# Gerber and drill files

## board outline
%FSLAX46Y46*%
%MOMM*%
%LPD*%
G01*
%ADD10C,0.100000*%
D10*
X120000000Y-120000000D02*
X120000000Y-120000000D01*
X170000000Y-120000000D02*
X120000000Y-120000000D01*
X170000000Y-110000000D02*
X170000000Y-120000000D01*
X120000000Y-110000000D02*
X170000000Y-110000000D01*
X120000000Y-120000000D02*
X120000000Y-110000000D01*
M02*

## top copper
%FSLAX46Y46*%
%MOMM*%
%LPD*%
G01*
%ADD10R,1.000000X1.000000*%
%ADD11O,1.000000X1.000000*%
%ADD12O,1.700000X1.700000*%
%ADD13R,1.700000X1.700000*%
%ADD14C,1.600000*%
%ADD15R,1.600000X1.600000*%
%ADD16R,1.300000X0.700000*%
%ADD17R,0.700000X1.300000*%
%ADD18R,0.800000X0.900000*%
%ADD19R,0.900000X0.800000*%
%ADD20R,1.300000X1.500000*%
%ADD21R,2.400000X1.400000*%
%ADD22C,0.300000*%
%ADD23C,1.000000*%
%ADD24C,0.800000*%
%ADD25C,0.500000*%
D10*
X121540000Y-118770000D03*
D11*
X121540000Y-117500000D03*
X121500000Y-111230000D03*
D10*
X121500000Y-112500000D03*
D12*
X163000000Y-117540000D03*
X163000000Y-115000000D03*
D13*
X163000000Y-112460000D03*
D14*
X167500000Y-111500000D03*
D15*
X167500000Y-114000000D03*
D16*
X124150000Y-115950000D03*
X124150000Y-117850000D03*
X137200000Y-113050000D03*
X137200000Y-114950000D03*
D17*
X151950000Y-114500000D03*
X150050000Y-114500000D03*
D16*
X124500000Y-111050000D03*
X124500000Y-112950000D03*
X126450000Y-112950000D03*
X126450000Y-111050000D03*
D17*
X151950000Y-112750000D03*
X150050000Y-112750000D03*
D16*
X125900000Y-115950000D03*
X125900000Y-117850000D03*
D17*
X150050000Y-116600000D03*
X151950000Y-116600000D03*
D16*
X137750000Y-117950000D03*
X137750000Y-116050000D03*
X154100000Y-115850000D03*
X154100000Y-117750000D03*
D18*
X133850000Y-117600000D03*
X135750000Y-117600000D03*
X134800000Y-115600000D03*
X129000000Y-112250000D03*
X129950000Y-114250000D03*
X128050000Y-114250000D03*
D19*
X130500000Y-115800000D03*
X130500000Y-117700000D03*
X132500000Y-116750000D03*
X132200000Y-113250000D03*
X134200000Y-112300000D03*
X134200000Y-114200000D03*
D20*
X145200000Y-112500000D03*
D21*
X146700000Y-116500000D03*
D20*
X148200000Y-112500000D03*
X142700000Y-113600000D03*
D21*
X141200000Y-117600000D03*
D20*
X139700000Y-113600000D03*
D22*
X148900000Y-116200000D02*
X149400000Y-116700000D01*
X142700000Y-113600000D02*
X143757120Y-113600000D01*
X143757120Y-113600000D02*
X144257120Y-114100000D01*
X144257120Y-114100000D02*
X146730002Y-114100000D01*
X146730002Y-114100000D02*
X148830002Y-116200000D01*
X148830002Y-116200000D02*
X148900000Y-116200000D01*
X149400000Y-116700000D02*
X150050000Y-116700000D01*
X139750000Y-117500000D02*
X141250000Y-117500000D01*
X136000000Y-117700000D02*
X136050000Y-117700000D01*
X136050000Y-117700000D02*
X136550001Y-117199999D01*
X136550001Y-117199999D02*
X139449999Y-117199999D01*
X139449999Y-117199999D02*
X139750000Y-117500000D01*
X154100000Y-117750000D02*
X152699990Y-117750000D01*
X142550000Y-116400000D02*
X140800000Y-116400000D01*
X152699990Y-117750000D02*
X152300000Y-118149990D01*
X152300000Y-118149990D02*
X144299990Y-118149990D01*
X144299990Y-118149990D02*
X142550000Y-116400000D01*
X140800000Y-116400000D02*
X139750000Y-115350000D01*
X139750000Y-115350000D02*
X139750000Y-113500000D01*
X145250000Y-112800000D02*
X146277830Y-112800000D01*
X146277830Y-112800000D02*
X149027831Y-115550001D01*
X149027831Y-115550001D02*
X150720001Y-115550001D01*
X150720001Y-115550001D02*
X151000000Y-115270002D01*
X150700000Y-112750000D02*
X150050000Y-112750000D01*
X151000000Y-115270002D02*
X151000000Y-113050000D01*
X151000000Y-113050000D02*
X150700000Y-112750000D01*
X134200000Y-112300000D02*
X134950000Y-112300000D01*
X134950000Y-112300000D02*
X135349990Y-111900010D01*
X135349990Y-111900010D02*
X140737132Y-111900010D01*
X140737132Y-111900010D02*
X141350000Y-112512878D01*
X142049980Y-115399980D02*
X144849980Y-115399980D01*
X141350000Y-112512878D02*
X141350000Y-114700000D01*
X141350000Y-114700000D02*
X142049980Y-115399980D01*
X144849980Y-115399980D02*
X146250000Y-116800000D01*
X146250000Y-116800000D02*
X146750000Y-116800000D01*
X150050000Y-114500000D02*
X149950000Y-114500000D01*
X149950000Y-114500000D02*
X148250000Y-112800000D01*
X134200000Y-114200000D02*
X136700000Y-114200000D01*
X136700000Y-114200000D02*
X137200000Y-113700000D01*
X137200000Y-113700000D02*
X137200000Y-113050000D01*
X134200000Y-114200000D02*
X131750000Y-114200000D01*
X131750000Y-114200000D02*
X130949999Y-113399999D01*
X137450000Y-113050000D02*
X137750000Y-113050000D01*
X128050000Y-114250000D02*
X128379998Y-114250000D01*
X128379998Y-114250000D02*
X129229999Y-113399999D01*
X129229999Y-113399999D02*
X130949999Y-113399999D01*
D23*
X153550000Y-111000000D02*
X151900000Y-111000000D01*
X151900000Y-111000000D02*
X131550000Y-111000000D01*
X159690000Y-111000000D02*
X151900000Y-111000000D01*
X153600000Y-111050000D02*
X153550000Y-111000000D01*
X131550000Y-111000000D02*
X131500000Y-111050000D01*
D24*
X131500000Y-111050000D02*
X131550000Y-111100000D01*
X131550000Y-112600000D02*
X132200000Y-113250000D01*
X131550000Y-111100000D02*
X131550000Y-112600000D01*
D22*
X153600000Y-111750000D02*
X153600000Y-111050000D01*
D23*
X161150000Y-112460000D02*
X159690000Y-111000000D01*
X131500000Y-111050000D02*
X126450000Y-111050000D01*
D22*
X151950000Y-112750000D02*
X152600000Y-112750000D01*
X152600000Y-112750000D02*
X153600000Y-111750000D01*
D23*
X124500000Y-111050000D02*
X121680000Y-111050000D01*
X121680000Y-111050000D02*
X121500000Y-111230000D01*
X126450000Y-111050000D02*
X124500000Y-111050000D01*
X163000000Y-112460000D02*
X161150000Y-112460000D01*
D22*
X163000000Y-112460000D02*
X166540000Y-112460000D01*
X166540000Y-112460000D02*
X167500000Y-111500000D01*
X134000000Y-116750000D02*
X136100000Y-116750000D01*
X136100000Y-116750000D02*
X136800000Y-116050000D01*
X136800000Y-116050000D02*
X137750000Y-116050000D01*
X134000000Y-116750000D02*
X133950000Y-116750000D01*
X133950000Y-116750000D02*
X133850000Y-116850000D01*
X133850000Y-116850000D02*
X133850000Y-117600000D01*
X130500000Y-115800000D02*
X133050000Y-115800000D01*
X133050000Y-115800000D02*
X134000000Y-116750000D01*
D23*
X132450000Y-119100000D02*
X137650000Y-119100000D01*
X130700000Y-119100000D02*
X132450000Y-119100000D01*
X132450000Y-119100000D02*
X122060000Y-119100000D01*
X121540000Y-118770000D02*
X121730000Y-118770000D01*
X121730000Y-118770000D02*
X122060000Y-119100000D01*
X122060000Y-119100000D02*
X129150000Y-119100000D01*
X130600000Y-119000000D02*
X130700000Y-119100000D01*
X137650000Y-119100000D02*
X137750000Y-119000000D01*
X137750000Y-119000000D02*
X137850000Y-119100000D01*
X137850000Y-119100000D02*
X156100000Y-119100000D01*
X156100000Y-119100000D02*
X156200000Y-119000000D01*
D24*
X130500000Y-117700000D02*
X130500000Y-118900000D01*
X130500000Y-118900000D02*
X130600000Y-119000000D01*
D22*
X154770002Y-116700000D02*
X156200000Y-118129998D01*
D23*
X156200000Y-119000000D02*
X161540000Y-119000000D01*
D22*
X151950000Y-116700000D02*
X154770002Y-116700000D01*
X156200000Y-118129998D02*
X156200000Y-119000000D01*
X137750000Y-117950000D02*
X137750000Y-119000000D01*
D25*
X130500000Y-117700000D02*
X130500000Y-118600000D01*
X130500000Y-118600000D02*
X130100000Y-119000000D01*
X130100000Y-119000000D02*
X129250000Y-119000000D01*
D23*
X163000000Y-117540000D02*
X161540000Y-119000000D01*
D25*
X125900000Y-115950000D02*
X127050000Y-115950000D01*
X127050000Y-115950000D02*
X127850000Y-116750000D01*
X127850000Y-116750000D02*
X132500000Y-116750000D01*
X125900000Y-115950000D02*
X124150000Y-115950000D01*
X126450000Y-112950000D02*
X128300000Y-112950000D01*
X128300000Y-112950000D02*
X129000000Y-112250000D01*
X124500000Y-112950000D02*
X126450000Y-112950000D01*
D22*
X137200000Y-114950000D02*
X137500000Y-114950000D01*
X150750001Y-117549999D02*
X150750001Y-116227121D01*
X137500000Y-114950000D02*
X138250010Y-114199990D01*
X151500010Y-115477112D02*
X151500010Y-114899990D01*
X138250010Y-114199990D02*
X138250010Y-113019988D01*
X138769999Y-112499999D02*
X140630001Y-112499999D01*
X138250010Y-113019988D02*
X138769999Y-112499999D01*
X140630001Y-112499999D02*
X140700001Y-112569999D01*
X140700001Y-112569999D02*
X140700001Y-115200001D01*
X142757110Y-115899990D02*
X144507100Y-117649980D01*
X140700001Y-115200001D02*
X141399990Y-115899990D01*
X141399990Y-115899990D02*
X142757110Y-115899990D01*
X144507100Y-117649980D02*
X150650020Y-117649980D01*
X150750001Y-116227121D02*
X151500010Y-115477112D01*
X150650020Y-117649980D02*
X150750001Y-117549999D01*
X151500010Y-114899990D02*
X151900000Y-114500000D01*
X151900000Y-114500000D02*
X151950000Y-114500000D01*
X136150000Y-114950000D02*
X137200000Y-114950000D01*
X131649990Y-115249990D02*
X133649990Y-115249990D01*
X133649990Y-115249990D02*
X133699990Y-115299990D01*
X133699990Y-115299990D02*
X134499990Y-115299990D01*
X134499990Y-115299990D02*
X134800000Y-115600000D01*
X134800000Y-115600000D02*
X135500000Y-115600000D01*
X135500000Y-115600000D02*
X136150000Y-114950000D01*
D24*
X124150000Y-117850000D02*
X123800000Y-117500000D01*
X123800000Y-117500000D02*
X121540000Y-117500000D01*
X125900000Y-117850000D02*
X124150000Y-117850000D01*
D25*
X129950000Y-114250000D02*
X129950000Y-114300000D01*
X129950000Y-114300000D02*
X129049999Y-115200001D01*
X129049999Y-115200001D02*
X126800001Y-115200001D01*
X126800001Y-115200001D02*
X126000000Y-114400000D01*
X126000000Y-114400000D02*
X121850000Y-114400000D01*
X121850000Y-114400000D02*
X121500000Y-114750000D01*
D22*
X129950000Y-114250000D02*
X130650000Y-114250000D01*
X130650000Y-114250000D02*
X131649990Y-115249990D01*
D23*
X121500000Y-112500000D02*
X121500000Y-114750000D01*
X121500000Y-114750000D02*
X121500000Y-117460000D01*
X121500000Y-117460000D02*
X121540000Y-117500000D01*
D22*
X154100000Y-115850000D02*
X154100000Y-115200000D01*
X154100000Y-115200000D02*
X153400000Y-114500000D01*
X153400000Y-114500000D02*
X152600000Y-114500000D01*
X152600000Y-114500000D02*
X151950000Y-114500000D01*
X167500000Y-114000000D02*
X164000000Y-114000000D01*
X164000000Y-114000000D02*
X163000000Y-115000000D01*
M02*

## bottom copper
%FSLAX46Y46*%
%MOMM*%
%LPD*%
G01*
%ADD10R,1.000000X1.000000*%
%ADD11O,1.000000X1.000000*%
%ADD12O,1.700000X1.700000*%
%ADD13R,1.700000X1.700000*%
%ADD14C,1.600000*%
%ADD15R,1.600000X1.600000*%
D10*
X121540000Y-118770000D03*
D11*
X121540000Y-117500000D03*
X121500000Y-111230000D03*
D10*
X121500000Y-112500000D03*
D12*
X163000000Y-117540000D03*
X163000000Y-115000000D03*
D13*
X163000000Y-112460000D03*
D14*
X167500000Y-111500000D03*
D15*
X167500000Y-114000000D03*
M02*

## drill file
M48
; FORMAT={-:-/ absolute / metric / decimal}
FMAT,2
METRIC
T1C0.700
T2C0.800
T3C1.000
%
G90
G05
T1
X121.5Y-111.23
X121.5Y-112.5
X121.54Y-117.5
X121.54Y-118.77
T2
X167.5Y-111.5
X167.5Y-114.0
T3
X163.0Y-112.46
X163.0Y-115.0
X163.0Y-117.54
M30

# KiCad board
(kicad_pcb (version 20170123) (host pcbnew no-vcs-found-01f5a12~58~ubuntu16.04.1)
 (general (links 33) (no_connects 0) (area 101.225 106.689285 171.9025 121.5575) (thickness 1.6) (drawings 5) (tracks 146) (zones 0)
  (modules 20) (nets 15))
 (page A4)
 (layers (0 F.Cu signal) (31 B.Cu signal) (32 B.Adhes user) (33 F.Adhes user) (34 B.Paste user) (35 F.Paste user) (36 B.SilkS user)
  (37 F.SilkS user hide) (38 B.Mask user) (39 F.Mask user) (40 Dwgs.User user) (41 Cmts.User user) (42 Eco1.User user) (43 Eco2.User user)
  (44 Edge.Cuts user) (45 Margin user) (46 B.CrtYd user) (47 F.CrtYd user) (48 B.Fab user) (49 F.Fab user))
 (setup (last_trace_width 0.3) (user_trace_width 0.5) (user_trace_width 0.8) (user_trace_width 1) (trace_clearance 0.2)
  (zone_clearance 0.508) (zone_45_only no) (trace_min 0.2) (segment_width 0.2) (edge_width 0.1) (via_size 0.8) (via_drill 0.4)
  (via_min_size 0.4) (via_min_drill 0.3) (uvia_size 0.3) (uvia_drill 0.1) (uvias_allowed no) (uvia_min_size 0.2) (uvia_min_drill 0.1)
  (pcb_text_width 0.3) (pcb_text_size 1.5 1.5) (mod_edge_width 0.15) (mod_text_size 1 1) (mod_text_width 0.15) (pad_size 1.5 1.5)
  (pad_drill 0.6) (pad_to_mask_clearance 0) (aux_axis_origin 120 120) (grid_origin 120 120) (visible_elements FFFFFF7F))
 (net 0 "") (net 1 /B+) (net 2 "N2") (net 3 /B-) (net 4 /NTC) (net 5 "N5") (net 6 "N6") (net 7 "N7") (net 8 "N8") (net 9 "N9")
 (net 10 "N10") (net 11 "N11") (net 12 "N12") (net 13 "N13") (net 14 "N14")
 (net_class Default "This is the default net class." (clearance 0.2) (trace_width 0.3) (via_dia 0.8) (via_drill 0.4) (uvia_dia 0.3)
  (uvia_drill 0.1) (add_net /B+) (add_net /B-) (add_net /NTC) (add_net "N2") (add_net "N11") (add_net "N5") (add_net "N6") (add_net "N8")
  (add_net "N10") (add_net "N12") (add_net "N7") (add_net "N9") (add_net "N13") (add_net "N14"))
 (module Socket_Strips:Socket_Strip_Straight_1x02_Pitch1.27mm (layer F.Cu) (at 121.54 118.77 180)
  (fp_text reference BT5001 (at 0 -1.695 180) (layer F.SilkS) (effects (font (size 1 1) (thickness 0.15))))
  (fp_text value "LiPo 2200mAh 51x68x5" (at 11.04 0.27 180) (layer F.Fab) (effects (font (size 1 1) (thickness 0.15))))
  (pad 1 thru_hole rect (at 0 0 180) (size 1 1) (drill 0.7) (layers *.Cu *.Mask) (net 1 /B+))
  (pad 2 thru_hole oval (at 0 1.27 180) (size 1 1) (drill 0.7) (layers *.Cu *.Mask) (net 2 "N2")))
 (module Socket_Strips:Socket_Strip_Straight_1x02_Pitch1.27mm (layer F.Cu) (at 121.5 112.5 180)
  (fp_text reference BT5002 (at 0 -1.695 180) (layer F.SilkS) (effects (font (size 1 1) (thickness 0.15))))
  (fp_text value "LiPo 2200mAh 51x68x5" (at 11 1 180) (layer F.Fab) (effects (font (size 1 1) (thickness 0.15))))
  (pad 2 thru_hole oval (at 0 1.27 180) (size 1 1) (drill 0.7) (layers *.Cu *.Mask) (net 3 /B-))
  (pad 1 thru_hole rect (at 0 0 180) (size 1 1) (drill 0.7) (layers *.Cu *.Mask) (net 2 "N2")))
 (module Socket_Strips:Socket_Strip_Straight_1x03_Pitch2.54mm (layer F.Cu) (at 163 112.46)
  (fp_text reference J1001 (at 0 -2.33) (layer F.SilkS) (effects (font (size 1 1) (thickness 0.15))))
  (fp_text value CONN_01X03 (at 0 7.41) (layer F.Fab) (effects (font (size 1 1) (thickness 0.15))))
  (pad 3 thru_hole oval (at 0 5.08) (size 1.7 1.7) (drill 1) (layers *.Cu *.Mask) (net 1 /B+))
  (pad 2 thru_hole oval (at 0 2.54) (size 1.7 1.7) (drill 1) (layers *.Cu *.Mask) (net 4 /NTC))
  (pad 1 thru_hole rect (at 0 0) (size 1.7 1.7) (drill 1) (layers *.Cu *.Mask) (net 3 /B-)))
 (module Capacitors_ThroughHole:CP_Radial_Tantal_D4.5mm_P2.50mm (layer F.Cu) (at 167.5 114 90)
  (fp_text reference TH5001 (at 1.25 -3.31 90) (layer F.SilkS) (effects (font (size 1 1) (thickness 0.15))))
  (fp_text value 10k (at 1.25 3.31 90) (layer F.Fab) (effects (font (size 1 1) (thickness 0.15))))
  (pad 2 thru_hole circle (at 2.5 0 90) (size 1.6 1.6) (drill 0.8) (layers *.Cu *.Mask) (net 3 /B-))
  (pad 1 thru_hole rect (at 0 0 90) (size 1.6 1.6) (drill 0.8) (layers *.Cu *.Mask) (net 4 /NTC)))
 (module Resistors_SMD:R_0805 (layer F.Cu) (at 124.15 116.9 270)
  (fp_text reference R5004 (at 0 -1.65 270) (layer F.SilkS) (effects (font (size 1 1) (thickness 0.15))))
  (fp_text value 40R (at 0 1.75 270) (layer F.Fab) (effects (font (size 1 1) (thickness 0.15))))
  (pad 1 smd rect (at -0.95 0 270) (size 0.7 1.3) (layers F.Cu F.Paste F.Mask) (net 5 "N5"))
  (pad 2 smd rect (at 0.95 0 270) (size 0.7 1.3) (layers F.Cu F.Paste F.Mask) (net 2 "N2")))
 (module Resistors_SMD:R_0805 (layer F.Cu) (at 137.2 114 90)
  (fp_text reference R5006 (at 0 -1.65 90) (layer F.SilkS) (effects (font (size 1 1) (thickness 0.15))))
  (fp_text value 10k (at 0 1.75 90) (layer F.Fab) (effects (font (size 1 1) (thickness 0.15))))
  (pad 2 smd rect (at 0.95 0 90) (size 0.7 1.3) (layers F.Cu F.Paste F.Mask) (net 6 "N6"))
  (pad 1 smd rect (at -0.95 0 90) (size 0.7 1.3) (layers F.Cu F.Paste F.Mask) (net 2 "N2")))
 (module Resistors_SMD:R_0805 (layer F.Cu) (at 151 114.5 180)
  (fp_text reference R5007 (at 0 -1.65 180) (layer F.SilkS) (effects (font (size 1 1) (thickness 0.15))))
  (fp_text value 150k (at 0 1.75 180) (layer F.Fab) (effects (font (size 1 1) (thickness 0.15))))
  (pad 1 smd rect (at -0.95 0 180) (size 0.7 1.3) (layers F.Cu F.Paste F.Mask) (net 2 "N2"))
  (pad 2 smd rect (at 0.95 0 180) (size 0.7 1.3) (layers F.Cu F.Paste F.Mask) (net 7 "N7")))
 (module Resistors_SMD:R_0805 (layer F.Cu) (at 124.5 112 90)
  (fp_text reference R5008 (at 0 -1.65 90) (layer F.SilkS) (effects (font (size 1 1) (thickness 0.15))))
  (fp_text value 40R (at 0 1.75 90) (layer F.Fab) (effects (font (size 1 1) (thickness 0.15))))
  (pad 2 smd rect (at 0.95 0 90) (size 0.7 1.3) (layers F.Cu F.Paste F.Mask) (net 3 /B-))
  (pad 1 smd rect (at -0.95 0 90) (size 0.7 1.3) (layers F.Cu F.Paste F.Mask) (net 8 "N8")))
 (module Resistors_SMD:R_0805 (layer F.Cu) (at 126.45 112 90)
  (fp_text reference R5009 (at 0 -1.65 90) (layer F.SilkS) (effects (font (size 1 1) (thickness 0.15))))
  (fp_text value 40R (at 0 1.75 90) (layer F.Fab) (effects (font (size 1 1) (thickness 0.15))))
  (pad 1 smd rect (at -0.95 0 90) (size 0.7 1.3) (layers F.Cu F.Paste F.Mask) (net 8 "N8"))
  (pad 2 smd rect (at 0.95 0 90) (size 0.7 1.3) (layers F.Cu F.Paste F.Mask) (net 3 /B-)))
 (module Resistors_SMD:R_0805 (layer F.Cu) (at 151 112.75)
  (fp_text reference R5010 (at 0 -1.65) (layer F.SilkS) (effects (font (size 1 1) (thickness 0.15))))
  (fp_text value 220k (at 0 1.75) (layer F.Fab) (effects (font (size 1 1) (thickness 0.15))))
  (pad 2 smd rect (at 0.95 0) (size 0.7 1.3) (layers F.Cu F.Paste F.Mask) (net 3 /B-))
  (pad 1 smd rect (at -0.95 0) (size 0.7 1.3) (layers F.Cu F.Paste F.Mask) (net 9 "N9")))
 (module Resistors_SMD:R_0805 (layer F.Cu) (at 125.9 116.9 270)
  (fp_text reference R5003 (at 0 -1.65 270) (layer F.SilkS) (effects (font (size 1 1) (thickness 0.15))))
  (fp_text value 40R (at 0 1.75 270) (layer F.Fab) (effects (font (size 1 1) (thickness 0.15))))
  (pad 1 smd rect (at -0.95 0 270) (size 0.7 1.3) (layers F.Cu F.Paste F.Mask) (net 5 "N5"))
  (pad 2 smd rect (at 0.95 0 270) (size 0.7 1.3) (layers F.Cu F.Paste F.Mask) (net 2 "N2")))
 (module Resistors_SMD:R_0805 (layer F.Cu) (at 151 116.6 180)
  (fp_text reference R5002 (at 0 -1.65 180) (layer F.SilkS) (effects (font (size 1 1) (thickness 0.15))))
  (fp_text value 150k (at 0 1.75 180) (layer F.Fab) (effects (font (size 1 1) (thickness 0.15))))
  (pad 2 smd rect (at 0.95 0 180) (size 0.7 1.3) (layers F.Cu F.Paste F.Mask) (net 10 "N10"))
  (pad 1 smd rect (at -0.95 0 180) (size 0.7 1.3) (layers F.Cu F.Paste F.Mask) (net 1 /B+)))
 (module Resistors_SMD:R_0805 (layer F.Cu) (at 137.75 117 90)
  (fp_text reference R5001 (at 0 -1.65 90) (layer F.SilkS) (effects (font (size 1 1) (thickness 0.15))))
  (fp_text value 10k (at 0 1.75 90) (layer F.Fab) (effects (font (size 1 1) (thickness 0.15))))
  (pad 1 smd rect (at -0.95 0 90) (size 0.7 1.3) (layers F.Cu F.Paste F.Mask) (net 1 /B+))
  (pad 2 smd rect (at 0.95 0 90) (size 0.7 1.3) (layers F.Cu F.Paste F.Mask) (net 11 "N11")))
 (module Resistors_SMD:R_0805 (layer F.Cu) (at 154.1 116.8 90)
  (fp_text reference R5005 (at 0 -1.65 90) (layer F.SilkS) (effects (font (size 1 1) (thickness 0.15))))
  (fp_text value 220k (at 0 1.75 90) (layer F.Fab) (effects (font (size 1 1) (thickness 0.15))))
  (pad 2 smd rect (at 0.95 0 90) (size 0.7 1.3) (layers F.Cu F.Paste F.Mask) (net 2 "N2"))
  (pad 1 smd rect (at -0.95 0 90) (size 0.7 1.3) (layers F.Cu F.Paste F.Mask) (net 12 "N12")))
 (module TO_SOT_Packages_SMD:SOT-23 (layer F.Cu) (at 134.8 116.6 90)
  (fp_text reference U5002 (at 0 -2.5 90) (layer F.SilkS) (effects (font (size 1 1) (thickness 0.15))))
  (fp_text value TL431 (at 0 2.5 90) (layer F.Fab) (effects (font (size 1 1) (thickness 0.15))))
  (pad 1 smd rect (at -1 -0.95 90) (size 0.9 0.8) (layers F.Cu F.Paste F.Mask) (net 11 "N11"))
  (pad 2 smd rect (at -1 0.95 90) (size 0.9 0.8) (layers F.Cu F.Paste F.Mask) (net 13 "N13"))
  (pad 3 smd rect (at 1 0 90) (size 0.9 0.8) (layers F.Cu F.Paste F.Mask) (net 2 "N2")))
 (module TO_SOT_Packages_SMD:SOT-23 (layer F.Cu) (at 129 113.25 90)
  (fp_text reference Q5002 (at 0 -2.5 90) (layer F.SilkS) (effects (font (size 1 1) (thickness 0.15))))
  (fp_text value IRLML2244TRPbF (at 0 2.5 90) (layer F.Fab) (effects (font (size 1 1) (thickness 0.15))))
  (pad 3 smd rect (at 1 0 90) (size 0.9 0.8) (layers F.Cu F.Paste F.Mask) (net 8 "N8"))
  (pad 2 smd rect (at -1 0.95 90) (size 0.9 0.8) (layers F.Cu F.Paste F.Mask) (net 2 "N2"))
  (pad 1 smd rect (at -1 -0.95 90) (size 0.9 0.8) (layers F.Cu F.Paste F.Mask) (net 6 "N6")))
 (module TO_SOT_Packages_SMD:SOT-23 (layer F.Cu) (at 131.5 116.75)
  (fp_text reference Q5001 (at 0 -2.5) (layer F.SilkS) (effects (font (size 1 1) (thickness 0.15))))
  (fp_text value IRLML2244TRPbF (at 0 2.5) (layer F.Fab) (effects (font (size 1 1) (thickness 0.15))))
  (pad 1 smd rect (at -1 -0.95) (size 0.9 0.8) (layers F.Cu F.Paste F.Mask) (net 11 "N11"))
  (pad 2 smd rect (at -1 0.95) (size 0.9 0.8) (layers F.Cu F.Paste F.Mask) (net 1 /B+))
  (pad 3 smd rect (at 1 0) (size 0.9 0.8) (layers F.Cu F.Paste F.Mask) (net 5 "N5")))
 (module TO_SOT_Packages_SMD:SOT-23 (layer F.Cu) (at 133.2 113.25 180)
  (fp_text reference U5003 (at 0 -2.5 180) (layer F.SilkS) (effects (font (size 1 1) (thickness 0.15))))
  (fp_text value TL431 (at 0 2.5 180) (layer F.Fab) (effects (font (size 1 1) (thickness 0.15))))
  (pad 3 smd rect (at 1 0 180) (size 0.9 0.8) (layers F.Cu F.Paste F.Mask) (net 3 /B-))
  (pad 2 smd rect (at -1 0.95 180) (size 0.9 0.8) (layers F.Cu F.Paste F.Mask) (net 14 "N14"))
  (pad 1 smd rect (at -1 -0.95 180) (size 0.9 0.8) (layers F.Cu F.Paste F.Mask) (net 6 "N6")))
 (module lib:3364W (layer F.Cu) (at 146.7 114.5 180)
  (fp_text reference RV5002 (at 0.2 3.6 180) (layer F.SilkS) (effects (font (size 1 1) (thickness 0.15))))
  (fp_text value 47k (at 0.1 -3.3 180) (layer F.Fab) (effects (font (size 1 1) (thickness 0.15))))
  (pad 3 smd rect (at 1.5 2 180) (size 1.3 1.5) (layers F.Cu F.Paste F.Mask) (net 9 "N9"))
  (pad 2 smd rect (at 0 -2 180) (size 2.4 1.4) (layers F.Cu F.Paste F.Mask) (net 14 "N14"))
  (pad 1 smd rect (at -1.5 2 180) (size 1.3 1.5) (layers F.Cu F.Paste F.Mask) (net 7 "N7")))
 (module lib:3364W (layer F.Cu) (at 141.2 115.6 180)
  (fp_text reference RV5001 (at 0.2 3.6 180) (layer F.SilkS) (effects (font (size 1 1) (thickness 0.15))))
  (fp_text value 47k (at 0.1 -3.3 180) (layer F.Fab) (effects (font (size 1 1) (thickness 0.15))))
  (pad 1 smd rect (at -1.5 2 180) (size 1.3 1.5) (layers F.Cu F.Paste F.Mask) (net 10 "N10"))
  (pad 2 smd rect (at 0 -2 180) (size 2.4 1.4) (layers F.Cu F.Paste F.Mask) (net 13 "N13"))
  (pad 3 smd rect (at 1.5 2 180) (size 1.3 1.5) (layers F.Cu F.Paste F.Mask) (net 12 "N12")))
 (gr_line (start 120 120) (end 120 120) (layer Edge.Cuts) (width 0.1))
 (gr_line (start 170 120) (end 120 120) (layer Edge.Cuts) (width 0.1))
 (gr_line (start 170 110) (end 170 120) (layer Edge.Cuts) (width 0.1))
 (gr_line (start 120 110) (end 170 110) (layer Edge.Cuts) (width 0.1))
 (gr_line (start 120 120) (end 120 110) (layer Edge.Cuts) (width 0.1))
 (segment (start 148.9 116.2) (end 149.4 116.7) (width 0.3) (layer F.Cu) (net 10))
 (segment (start 142.7 113.6) (end 143.75712 113.6) (width 0.3) (layer F.Cu) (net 10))
 (segment (start 143.75712 113.6) (end 144.25712 114.1) (width 0.3) (layer F.Cu) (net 10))
 (segment (start 144.25712 114.1) (end 146.730002 114.1) (width 0.3) (layer F.Cu) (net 10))
 (segment (start 146.730002 114.1) (end 148.830002 116.2) (width 0.3) (layer F.Cu) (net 10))
 (segment (start 148.830002 116.2) (end 148.9 116.2) (width 0.3) (layer F.Cu) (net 10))
 (segment (start 149.4 116.7) (end 150.05 116.7) (width 0.3) (layer F.Cu) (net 10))
 (segment (start 139.75 117.5) (end 141.25 117.5) (width 0.3) (layer F.Cu) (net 13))
 (segment (start 136 117.7) (end 136.05 117.7) (width 0.3) (layer F.Cu) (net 13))
 (segment (start 136.05 117.7) (end 136.550001 117.199999) (width 0.3) (layer F.Cu) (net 13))
 (segment (start 136.550001 117.199999) (end 139.449999 117.199999) (width 0.3) (layer F.Cu) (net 13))
 (segment (start 139.449999 117.199999) (end 139.75 117.5) (width 0.3) (layer F.Cu) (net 13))
 (segment (start 154.1 117.75) (end 152.69999 117.75) (width 0.3) (layer F.Cu) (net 12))
 (segment (start 142.55 116.4) (end 140.8 116.4) (width 0.3) (layer F.Cu) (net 12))
 (segment (start 152.69999 117.75) (end 152.3 118.14999) (width 0.3) (layer F.Cu) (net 12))
 (segment (start 152.3 118.14999) (end 144.29999 118.14999) (width 0.3) (layer F.Cu) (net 12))
 (segment (start 144.29999 118.14999) (end 142.55 116.4) (width 0.3) (layer F.Cu) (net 12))
 (segment (start 140.8 116.4) (end 139.75 115.35) (width 0.3) (layer F.Cu) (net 12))
 (segment (start 139.75 115.35) (end 139.75 113.5) (width 0.3) (layer F.Cu) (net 12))
 (segment (start 145.25 112.8) (end 146.27783 112.8) (width 0.3) (layer F.Cu) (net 9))
 (segment (start 146.27783 112.8) (end 149.027831 115.550001) (width 0.3) (layer F.Cu) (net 9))
 (segment (start 149.027831 115.550001) (end 150.720001 115.550001) (width 0.3) (layer F.Cu) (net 9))
 (segment (start 150.720001 115.550001) (end 151 115.270002) (width 0.3) (layer F.Cu) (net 9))
 (segment (start 150.7 112.75) (end 150.05 112.75) (width 0.3) (layer F.Cu) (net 9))
 (segment (start 151 115.270002) (end 151 113.05) (width 0.3) (layer F.Cu) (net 9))
 (segment (start 151 113.05) (end 150.7 112.75) (width 0.3) (layer F.Cu) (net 9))
 (segment (start 134.2 112.3) (end 134.95 112.3) (width 0.3) (layer F.Cu) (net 14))
 (segment (start 134.95 112.3) (end 135.34999 111.90001) (width 0.3) (layer F.Cu) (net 14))
 (segment (start 135.34999 111.90001) (end 140.737132 111.90001) (width 0.3) (layer F.Cu) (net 14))
 (segment (start 140.737132 111.90001) (end 141.35 112.512878) (width 0.3) (layer F.Cu) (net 14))
 (segment (start 142.04998 115.39998) (end 144.84998 115.39998) (width 0.3) (layer F.Cu) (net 14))
 (segment (start 141.35 112.512878) (end 141.35 114.7) (width 0.3) (layer F.Cu) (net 14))
 (segment (start 141.35 114.7) (end 142.04998 115.39998) (width 0.3) (layer F.Cu) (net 14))
 (segment (start 144.84998 115.39998) (end 146.25 116.8) (width 0.3) (layer F.Cu) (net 14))
 (segment (start 146.25 116.8) (end 146.75 116.8) (width 0.3) (layer F.Cu) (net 14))
 (segment (start 150.05 114.5) (end 149.95 114.5) (width 0.3) (layer F.Cu) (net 7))
 (segment (start 149.95 114.5) (end 148.25 112.8) (width 0.3) (layer F.Cu) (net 7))
 (segment (start 134.2 114.2) (end 136.7 114.2) (width 0.3) (layer F.Cu) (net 6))
 (segment (start 136.7 114.2) (end 137.2 113.7) (width 0.3) (layer F.Cu) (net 6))
 (segment (start 137.2 113.7) (end 137.2 113.05) (width 0.3) (layer F.Cu) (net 6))
 (segment (start 134.2 114.2) (end 131.75 114.2) (width 0.3) (layer F.Cu) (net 6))
 (segment (start 131.75 114.2) (end 130.949999 113.399999) (width 0.3) (layer F.Cu) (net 6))
 (segment (start 137.45 113.05) (end 137.75 113.05) (width 0.3) (layer F.Cu) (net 6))
 (segment (start 128.05 114.25) (end 128.379998 114.25) (width 0.3) (layer F.Cu) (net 6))
 (segment (start 128.379998 114.25) (end 129.229999 113.399999) (width 0.3) (layer F.Cu) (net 6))
 (segment (start 129.229999 113.399999) (end 130.949999 113.399999) (width 0.3) (layer F.Cu) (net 6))
 (segment (start 153.55 111) (end 151.9 111) (width 1) (layer F.Cu) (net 3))
 (segment (start 151.9 111) (end 131.55 111) (width 1) (layer F.Cu) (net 3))
 (segment (start 159.69 111) (end 151.9 111) (width 1) (layer F.Cu) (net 3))
 (segment (start 153.6 111.05) (end 153.55 111) (width 1) (layer F.Cu) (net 3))
 (segment (start 131.55 111) (end 131.5 111.05) (width 1) (layer F.Cu) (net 3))
 (segment (start 131.5 111.05) (end 131.55 111.1) (width 0.8) (layer F.Cu) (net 3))
 (segment (start 131.55 112.6) (end 132.2 113.25) (width 0.8) (layer F.Cu) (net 3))
 (segment (start 131.55 111.1) (end 131.55 112.6) (width 0.8) (layer F.Cu) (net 3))
 (segment (start 153.6 111.75) (end 153.6 111.05) (width 0.3) (layer F.Cu) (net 3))
 (segment (start 161.15 112.46) (end 159.69 111) (width 1) (layer F.Cu) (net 3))
 (segment (start 131.5 111.05) (end 126.45 111.05) (width 1) (layer F.Cu) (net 3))
 (segment (start 151.95 112.75) (end 152.6 112.75) (width 0.3) (layer F.Cu) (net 3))
 (segment (start 152.6 112.75) (end 153.6 111.75) (width 0.3) (layer F.Cu) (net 3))
 (segment (start 124.5 111.05) (end 121.68 111.05) (width 1) (layer F.Cu) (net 3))
 (segment (start 121.68 111.05) (end 121.5 111.23) (width 1) (layer F.Cu) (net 3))
 (segment (start 126.45 111.05) (end 124.5 111.05) (width 1) (layer F.Cu) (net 3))
 (segment (start 163 112.46) (end 161.15 112.46) (width 1) (layer F.Cu) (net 3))
 (segment (start 163 112.46) (end 166.54 112.46) (width 0.3) (layer F.Cu) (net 3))
 (segment (start 166.54 112.46) (end 167.5 111.5) (width 0.3) (layer F.Cu) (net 3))
 (segment (start 134 116.75) (end 136.1 116.75) (width 0.3) (layer F.Cu) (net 11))
 (segment (start 136.1 116.75) (end 136.8 116.05) (width 0.3) (layer F.Cu) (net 11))
 (segment (start 136.8 116.05) (end 137.75 116.05) (width 0.3) (layer F.Cu) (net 11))
 (segment (start 134 116.75) (end 133.95 116.75) (width 0.3) (layer F.Cu) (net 11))
 (segment (start 133.95 116.75) (end 133.85 116.85) (width 0.3) (layer F.Cu) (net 11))
 (segment (start 133.85 116.85) (end 133.85 117.6) (width 0.3) (layer F.Cu) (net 11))
 (segment (start 130.5 115.8) (end 133.05 115.8) (width 0.3) (layer F.Cu) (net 11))
 (segment (start 133.05 115.8) (end 134 116.75) (width 0.3) (layer F.Cu) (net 11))
 (segment (start 132.45 119.1) (end 137.65 119.1) (width 1) (layer F.Cu) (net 1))
 (segment (start 130.7 119.1) (end 132.45 119.1) (width 1) (layer F.Cu) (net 1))
 (segment (start 132.45 119.1) (end 122.06 119.1) (width 1) (layer F.Cu) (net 1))
 (segment (start 121.54 118.77) (end 121.73 118.77) (width 1) (layer F.Cu) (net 1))
 (segment (start 121.73 118.77) (end 122.06 119.1) (width 1) (layer F.Cu) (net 1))
 (segment (start 122.06 119.1) (end 129.15 119.1) (width 1) (layer F.Cu) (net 1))
 (segment (start 130.6 119) (end 130.7 119.1) (width 1) (layer F.Cu) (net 1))
 (segment (start 137.65 119.1) (end 137.75 119) (width 1) (layer F.Cu) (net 1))
 (segment (start 137.75 119) (end 137.85 119.1) (width 1) (layer F.Cu) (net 1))
 (segment (start 137.85 119.1) (end 156.1 119.1) (width 1) (layer F.Cu) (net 1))
 (segment (start 156.1 119.1) (end 156.2 119) (width 1) (layer F.Cu) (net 1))
 (segment (start 130.5 117.7) (end 130.5 118.9) (width 0.8) (layer F.Cu) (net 1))
 (segment (start 130.5 118.9) (end 130.6 119) (width 0.8) (layer F.Cu) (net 1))
 (segment (start 154.770002 116.7) (end 156.2 118.129998) (width 0.3) (layer F.Cu) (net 1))
 (segment (start 156.2 119) (end 161.54 119) (width 1) (layer F.Cu) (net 1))
 (segment (start 151.95 116.7) (end 154.770002 116.7) (width 0.3) (layer F.Cu) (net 1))
 (segment (start 156.2 118.129998) (end 156.2 119) (width 0.3) (layer F.Cu) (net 1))
 (segment (start 137.75 117.95) (end 137.75 119) (width 0.3) (layer F.Cu) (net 1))
 (segment (start 130.5 117.7) (end 130.5 118.6) (width 0.5) (layer F.Cu) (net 1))
 (segment (start 130.5 118.6) (end 130.1 119) (width 0.5) (layer F.Cu) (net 1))
 (segment (start 130.1 119) (end 129.25 119) (width 0.5) (layer F.Cu) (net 1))
 (segment (start 163 117.54) (end 161.54 119) (width 1) (layer F.Cu) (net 1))
 (segment (start 125.9 115.95) (end 127.05 115.95) (width 0.5) (layer F.Cu) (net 5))
 (segment (start 127.05 115.95) (end 127.85 116.75) (width 0.5) (layer F.Cu) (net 5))
 (segment (start 127.85 116.75) (end 132.5 116.75) (width 0.5) (layer F.Cu) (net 5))
 (segment (start 125.9 115.95) (end 124.15 115.95) (width 0.5) (layer F.Cu) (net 5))
 (segment (start 126.45 112.95) (end 128.3 112.95) (width 0.5) (layer F.Cu) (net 8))
 (segment (start 128.3 112.95) (end 129 112.25) (width 0.5) (layer F.Cu) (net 8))
 (segment (start 124.5 112.95) (end 126.45 112.95) (width 0.5) (layer F.Cu) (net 8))
 (segment (start 137.2 114.95) (end 137.5 114.95) (width 0.3) (layer F.Cu) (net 2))
 (segment (start 150.750001 117.549999) (end 150.750001 116.227121) (width 0.3) (layer F.Cu) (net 2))
 (segment (start 137.5 114.95) (end 138.25001 114.19999) (width 0.3) (layer F.Cu) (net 2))
 (segment (start 151.50001 115.477112) (end 151.50001 114.89999) (width 0.3) (layer F.Cu) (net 2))
 (segment (start 138.25001 114.19999) (end 138.25001 113.019988) (width 0.3) (layer F.Cu) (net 2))
 (segment (start 138.769999 112.499999) (end 140.630001 112.499999) (width 0.3) (layer F.Cu) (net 2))
 (segment (start 138.25001 113.019988) (end 138.769999 112.499999) (width 0.3) (layer F.Cu) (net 2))
 (segment (start 140.630001 112.499999) (end 140.700001 112.569999) (width 0.3) (layer F.Cu) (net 2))
 (segment (start 140.700001 112.569999) (end 140.700001 115.200001) (width 0.3) (layer F.Cu) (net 2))
 (segment (start 142.75711 115.89999) (end 144.5071 117.64998) (width 0.3) (layer F.Cu) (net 2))
 (segment (start 140.700001 115.200001) (end 141.39999 115.89999) (width 0.3) (layer F.Cu) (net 2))
 (segment (start 141.39999 115.89999) (end 142.75711 115.89999) (width 0.3) (layer F.Cu) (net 2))
 (segment (start 144.5071 117.64998) (end 150.65002 117.64998) (width 0.3) (layer F.Cu) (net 2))
 (segment (start 150.750001 116.227121) (end 151.50001 115.477112) (width 0.3) (layer F.Cu) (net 2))
 (segment (start 150.65002 117.64998) (end 150.750001 117.549999) (width 0.3) (layer F.Cu) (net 2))
 (segment (start 151.50001 114.89999) (end 151.9 114.5) (width 0.3) (layer F.Cu) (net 2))
 (segment (start 151.9 114.5) (end 151.95 114.5) (width 0.3) (layer F.Cu) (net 2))
 (segment (start 136.15 114.95) (end 137.2 114.95) (width 0.3) (layer F.Cu) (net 2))
 (segment (start 131.64999 115.24999) (end 133.64999 115.24999) (width 0.3) (layer F.Cu) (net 2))
 (segment (start 133.64999 115.24999) (end 133.69999 115.29999) (width 0.3) (layer F.Cu) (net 2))
 (segment (start 133.69999 115.29999) (end 134.49999 115.29999) (width 0.3) (layer F.Cu) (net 2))
 (segment (start 134.49999 115.29999) (end 134.8 115.6) (width 0.3) (layer F.Cu) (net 2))
 (segment (start 134.8 115.6) (end 135.5 115.6) (width 0.3) (layer F.Cu) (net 2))
 (segment (start 135.5 115.6) (end 136.15 114.95) (width 0.3) (layer F.Cu) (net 2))
 (segment (start 124.15 117.85) (end 123.8 117.5) (width 0.8) (layer F.Cu) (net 2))
 (segment (start 123.8 117.5) (end 121.54 117.5) (width 0.8) (layer F.Cu) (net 2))
 (segment (start 125.9 117.85) (end 124.15 117.85) (width 0.8) (layer F.Cu) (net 2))
 (segment (start 129.95 114.25) (end 129.95 114.3) (width 0.5) (layer F.Cu) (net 2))
 (segment (start 129.95 114.3) (end 129.049999 115.200001) (width 0.5) (layer F.Cu) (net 2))
 (segment (start 129.049999 115.200001) (end 126.800001 115.200001) (width 0.5) (layer F.Cu) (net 2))
 (segment (start 126.800001 115.200001) (end 126 114.4) (width 0.5) (layer F.Cu) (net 2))
 (segment (start 126 114.4) (end 121.85 114.4) (width 0.5) (layer F.Cu) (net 2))
 (segment (start 121.85 114.4) (end 121.5 114.75) (width 0.5) (layer F.Cu) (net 2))
 (segment (start 129.95 114.25) (end 130.65 114.25) (width 0.3) (layer F.Cu) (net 2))
 (segment (start 130.65 114.25) (end 131.64999 115.24999) (width 0.3) (layer F.Cu) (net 2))
 (segment (start 121.5 112.5) (end 121.5 114.75) (width 1) (layer F.Cu) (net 2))
 (segment (start 121.5 114.75) (end 121.5 117.46) (width 1) (layer F.Cu) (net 2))
 (segment (start 121.5 117.46) (end 121.54 117.5) (width 1) (layer F.Cu) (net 2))
 (segment (start 154.1 115.85) (end 154.1 115.2) (width 0.3) (layer F.Cu) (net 2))
 (segment (start 154.1 115.2) (end 153.4 114.5) (width 0.3) (layer F.Cu) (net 2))
 (segment (start 153.4 114.5) (end 152.6 114.5) (width 0.3) (layer F.Cu) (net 2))
 (segment (start 152.6 114.5) (end 151.95 114.5) (width 0.3) (layer F.Cu) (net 2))
 (segment (start 167.5 114) (end 164 114) (width 0.3) (layer F.Cu) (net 4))
 (segment (start 164 114) (end 163 115) (width 0.3) (layer F.Cu) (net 4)))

